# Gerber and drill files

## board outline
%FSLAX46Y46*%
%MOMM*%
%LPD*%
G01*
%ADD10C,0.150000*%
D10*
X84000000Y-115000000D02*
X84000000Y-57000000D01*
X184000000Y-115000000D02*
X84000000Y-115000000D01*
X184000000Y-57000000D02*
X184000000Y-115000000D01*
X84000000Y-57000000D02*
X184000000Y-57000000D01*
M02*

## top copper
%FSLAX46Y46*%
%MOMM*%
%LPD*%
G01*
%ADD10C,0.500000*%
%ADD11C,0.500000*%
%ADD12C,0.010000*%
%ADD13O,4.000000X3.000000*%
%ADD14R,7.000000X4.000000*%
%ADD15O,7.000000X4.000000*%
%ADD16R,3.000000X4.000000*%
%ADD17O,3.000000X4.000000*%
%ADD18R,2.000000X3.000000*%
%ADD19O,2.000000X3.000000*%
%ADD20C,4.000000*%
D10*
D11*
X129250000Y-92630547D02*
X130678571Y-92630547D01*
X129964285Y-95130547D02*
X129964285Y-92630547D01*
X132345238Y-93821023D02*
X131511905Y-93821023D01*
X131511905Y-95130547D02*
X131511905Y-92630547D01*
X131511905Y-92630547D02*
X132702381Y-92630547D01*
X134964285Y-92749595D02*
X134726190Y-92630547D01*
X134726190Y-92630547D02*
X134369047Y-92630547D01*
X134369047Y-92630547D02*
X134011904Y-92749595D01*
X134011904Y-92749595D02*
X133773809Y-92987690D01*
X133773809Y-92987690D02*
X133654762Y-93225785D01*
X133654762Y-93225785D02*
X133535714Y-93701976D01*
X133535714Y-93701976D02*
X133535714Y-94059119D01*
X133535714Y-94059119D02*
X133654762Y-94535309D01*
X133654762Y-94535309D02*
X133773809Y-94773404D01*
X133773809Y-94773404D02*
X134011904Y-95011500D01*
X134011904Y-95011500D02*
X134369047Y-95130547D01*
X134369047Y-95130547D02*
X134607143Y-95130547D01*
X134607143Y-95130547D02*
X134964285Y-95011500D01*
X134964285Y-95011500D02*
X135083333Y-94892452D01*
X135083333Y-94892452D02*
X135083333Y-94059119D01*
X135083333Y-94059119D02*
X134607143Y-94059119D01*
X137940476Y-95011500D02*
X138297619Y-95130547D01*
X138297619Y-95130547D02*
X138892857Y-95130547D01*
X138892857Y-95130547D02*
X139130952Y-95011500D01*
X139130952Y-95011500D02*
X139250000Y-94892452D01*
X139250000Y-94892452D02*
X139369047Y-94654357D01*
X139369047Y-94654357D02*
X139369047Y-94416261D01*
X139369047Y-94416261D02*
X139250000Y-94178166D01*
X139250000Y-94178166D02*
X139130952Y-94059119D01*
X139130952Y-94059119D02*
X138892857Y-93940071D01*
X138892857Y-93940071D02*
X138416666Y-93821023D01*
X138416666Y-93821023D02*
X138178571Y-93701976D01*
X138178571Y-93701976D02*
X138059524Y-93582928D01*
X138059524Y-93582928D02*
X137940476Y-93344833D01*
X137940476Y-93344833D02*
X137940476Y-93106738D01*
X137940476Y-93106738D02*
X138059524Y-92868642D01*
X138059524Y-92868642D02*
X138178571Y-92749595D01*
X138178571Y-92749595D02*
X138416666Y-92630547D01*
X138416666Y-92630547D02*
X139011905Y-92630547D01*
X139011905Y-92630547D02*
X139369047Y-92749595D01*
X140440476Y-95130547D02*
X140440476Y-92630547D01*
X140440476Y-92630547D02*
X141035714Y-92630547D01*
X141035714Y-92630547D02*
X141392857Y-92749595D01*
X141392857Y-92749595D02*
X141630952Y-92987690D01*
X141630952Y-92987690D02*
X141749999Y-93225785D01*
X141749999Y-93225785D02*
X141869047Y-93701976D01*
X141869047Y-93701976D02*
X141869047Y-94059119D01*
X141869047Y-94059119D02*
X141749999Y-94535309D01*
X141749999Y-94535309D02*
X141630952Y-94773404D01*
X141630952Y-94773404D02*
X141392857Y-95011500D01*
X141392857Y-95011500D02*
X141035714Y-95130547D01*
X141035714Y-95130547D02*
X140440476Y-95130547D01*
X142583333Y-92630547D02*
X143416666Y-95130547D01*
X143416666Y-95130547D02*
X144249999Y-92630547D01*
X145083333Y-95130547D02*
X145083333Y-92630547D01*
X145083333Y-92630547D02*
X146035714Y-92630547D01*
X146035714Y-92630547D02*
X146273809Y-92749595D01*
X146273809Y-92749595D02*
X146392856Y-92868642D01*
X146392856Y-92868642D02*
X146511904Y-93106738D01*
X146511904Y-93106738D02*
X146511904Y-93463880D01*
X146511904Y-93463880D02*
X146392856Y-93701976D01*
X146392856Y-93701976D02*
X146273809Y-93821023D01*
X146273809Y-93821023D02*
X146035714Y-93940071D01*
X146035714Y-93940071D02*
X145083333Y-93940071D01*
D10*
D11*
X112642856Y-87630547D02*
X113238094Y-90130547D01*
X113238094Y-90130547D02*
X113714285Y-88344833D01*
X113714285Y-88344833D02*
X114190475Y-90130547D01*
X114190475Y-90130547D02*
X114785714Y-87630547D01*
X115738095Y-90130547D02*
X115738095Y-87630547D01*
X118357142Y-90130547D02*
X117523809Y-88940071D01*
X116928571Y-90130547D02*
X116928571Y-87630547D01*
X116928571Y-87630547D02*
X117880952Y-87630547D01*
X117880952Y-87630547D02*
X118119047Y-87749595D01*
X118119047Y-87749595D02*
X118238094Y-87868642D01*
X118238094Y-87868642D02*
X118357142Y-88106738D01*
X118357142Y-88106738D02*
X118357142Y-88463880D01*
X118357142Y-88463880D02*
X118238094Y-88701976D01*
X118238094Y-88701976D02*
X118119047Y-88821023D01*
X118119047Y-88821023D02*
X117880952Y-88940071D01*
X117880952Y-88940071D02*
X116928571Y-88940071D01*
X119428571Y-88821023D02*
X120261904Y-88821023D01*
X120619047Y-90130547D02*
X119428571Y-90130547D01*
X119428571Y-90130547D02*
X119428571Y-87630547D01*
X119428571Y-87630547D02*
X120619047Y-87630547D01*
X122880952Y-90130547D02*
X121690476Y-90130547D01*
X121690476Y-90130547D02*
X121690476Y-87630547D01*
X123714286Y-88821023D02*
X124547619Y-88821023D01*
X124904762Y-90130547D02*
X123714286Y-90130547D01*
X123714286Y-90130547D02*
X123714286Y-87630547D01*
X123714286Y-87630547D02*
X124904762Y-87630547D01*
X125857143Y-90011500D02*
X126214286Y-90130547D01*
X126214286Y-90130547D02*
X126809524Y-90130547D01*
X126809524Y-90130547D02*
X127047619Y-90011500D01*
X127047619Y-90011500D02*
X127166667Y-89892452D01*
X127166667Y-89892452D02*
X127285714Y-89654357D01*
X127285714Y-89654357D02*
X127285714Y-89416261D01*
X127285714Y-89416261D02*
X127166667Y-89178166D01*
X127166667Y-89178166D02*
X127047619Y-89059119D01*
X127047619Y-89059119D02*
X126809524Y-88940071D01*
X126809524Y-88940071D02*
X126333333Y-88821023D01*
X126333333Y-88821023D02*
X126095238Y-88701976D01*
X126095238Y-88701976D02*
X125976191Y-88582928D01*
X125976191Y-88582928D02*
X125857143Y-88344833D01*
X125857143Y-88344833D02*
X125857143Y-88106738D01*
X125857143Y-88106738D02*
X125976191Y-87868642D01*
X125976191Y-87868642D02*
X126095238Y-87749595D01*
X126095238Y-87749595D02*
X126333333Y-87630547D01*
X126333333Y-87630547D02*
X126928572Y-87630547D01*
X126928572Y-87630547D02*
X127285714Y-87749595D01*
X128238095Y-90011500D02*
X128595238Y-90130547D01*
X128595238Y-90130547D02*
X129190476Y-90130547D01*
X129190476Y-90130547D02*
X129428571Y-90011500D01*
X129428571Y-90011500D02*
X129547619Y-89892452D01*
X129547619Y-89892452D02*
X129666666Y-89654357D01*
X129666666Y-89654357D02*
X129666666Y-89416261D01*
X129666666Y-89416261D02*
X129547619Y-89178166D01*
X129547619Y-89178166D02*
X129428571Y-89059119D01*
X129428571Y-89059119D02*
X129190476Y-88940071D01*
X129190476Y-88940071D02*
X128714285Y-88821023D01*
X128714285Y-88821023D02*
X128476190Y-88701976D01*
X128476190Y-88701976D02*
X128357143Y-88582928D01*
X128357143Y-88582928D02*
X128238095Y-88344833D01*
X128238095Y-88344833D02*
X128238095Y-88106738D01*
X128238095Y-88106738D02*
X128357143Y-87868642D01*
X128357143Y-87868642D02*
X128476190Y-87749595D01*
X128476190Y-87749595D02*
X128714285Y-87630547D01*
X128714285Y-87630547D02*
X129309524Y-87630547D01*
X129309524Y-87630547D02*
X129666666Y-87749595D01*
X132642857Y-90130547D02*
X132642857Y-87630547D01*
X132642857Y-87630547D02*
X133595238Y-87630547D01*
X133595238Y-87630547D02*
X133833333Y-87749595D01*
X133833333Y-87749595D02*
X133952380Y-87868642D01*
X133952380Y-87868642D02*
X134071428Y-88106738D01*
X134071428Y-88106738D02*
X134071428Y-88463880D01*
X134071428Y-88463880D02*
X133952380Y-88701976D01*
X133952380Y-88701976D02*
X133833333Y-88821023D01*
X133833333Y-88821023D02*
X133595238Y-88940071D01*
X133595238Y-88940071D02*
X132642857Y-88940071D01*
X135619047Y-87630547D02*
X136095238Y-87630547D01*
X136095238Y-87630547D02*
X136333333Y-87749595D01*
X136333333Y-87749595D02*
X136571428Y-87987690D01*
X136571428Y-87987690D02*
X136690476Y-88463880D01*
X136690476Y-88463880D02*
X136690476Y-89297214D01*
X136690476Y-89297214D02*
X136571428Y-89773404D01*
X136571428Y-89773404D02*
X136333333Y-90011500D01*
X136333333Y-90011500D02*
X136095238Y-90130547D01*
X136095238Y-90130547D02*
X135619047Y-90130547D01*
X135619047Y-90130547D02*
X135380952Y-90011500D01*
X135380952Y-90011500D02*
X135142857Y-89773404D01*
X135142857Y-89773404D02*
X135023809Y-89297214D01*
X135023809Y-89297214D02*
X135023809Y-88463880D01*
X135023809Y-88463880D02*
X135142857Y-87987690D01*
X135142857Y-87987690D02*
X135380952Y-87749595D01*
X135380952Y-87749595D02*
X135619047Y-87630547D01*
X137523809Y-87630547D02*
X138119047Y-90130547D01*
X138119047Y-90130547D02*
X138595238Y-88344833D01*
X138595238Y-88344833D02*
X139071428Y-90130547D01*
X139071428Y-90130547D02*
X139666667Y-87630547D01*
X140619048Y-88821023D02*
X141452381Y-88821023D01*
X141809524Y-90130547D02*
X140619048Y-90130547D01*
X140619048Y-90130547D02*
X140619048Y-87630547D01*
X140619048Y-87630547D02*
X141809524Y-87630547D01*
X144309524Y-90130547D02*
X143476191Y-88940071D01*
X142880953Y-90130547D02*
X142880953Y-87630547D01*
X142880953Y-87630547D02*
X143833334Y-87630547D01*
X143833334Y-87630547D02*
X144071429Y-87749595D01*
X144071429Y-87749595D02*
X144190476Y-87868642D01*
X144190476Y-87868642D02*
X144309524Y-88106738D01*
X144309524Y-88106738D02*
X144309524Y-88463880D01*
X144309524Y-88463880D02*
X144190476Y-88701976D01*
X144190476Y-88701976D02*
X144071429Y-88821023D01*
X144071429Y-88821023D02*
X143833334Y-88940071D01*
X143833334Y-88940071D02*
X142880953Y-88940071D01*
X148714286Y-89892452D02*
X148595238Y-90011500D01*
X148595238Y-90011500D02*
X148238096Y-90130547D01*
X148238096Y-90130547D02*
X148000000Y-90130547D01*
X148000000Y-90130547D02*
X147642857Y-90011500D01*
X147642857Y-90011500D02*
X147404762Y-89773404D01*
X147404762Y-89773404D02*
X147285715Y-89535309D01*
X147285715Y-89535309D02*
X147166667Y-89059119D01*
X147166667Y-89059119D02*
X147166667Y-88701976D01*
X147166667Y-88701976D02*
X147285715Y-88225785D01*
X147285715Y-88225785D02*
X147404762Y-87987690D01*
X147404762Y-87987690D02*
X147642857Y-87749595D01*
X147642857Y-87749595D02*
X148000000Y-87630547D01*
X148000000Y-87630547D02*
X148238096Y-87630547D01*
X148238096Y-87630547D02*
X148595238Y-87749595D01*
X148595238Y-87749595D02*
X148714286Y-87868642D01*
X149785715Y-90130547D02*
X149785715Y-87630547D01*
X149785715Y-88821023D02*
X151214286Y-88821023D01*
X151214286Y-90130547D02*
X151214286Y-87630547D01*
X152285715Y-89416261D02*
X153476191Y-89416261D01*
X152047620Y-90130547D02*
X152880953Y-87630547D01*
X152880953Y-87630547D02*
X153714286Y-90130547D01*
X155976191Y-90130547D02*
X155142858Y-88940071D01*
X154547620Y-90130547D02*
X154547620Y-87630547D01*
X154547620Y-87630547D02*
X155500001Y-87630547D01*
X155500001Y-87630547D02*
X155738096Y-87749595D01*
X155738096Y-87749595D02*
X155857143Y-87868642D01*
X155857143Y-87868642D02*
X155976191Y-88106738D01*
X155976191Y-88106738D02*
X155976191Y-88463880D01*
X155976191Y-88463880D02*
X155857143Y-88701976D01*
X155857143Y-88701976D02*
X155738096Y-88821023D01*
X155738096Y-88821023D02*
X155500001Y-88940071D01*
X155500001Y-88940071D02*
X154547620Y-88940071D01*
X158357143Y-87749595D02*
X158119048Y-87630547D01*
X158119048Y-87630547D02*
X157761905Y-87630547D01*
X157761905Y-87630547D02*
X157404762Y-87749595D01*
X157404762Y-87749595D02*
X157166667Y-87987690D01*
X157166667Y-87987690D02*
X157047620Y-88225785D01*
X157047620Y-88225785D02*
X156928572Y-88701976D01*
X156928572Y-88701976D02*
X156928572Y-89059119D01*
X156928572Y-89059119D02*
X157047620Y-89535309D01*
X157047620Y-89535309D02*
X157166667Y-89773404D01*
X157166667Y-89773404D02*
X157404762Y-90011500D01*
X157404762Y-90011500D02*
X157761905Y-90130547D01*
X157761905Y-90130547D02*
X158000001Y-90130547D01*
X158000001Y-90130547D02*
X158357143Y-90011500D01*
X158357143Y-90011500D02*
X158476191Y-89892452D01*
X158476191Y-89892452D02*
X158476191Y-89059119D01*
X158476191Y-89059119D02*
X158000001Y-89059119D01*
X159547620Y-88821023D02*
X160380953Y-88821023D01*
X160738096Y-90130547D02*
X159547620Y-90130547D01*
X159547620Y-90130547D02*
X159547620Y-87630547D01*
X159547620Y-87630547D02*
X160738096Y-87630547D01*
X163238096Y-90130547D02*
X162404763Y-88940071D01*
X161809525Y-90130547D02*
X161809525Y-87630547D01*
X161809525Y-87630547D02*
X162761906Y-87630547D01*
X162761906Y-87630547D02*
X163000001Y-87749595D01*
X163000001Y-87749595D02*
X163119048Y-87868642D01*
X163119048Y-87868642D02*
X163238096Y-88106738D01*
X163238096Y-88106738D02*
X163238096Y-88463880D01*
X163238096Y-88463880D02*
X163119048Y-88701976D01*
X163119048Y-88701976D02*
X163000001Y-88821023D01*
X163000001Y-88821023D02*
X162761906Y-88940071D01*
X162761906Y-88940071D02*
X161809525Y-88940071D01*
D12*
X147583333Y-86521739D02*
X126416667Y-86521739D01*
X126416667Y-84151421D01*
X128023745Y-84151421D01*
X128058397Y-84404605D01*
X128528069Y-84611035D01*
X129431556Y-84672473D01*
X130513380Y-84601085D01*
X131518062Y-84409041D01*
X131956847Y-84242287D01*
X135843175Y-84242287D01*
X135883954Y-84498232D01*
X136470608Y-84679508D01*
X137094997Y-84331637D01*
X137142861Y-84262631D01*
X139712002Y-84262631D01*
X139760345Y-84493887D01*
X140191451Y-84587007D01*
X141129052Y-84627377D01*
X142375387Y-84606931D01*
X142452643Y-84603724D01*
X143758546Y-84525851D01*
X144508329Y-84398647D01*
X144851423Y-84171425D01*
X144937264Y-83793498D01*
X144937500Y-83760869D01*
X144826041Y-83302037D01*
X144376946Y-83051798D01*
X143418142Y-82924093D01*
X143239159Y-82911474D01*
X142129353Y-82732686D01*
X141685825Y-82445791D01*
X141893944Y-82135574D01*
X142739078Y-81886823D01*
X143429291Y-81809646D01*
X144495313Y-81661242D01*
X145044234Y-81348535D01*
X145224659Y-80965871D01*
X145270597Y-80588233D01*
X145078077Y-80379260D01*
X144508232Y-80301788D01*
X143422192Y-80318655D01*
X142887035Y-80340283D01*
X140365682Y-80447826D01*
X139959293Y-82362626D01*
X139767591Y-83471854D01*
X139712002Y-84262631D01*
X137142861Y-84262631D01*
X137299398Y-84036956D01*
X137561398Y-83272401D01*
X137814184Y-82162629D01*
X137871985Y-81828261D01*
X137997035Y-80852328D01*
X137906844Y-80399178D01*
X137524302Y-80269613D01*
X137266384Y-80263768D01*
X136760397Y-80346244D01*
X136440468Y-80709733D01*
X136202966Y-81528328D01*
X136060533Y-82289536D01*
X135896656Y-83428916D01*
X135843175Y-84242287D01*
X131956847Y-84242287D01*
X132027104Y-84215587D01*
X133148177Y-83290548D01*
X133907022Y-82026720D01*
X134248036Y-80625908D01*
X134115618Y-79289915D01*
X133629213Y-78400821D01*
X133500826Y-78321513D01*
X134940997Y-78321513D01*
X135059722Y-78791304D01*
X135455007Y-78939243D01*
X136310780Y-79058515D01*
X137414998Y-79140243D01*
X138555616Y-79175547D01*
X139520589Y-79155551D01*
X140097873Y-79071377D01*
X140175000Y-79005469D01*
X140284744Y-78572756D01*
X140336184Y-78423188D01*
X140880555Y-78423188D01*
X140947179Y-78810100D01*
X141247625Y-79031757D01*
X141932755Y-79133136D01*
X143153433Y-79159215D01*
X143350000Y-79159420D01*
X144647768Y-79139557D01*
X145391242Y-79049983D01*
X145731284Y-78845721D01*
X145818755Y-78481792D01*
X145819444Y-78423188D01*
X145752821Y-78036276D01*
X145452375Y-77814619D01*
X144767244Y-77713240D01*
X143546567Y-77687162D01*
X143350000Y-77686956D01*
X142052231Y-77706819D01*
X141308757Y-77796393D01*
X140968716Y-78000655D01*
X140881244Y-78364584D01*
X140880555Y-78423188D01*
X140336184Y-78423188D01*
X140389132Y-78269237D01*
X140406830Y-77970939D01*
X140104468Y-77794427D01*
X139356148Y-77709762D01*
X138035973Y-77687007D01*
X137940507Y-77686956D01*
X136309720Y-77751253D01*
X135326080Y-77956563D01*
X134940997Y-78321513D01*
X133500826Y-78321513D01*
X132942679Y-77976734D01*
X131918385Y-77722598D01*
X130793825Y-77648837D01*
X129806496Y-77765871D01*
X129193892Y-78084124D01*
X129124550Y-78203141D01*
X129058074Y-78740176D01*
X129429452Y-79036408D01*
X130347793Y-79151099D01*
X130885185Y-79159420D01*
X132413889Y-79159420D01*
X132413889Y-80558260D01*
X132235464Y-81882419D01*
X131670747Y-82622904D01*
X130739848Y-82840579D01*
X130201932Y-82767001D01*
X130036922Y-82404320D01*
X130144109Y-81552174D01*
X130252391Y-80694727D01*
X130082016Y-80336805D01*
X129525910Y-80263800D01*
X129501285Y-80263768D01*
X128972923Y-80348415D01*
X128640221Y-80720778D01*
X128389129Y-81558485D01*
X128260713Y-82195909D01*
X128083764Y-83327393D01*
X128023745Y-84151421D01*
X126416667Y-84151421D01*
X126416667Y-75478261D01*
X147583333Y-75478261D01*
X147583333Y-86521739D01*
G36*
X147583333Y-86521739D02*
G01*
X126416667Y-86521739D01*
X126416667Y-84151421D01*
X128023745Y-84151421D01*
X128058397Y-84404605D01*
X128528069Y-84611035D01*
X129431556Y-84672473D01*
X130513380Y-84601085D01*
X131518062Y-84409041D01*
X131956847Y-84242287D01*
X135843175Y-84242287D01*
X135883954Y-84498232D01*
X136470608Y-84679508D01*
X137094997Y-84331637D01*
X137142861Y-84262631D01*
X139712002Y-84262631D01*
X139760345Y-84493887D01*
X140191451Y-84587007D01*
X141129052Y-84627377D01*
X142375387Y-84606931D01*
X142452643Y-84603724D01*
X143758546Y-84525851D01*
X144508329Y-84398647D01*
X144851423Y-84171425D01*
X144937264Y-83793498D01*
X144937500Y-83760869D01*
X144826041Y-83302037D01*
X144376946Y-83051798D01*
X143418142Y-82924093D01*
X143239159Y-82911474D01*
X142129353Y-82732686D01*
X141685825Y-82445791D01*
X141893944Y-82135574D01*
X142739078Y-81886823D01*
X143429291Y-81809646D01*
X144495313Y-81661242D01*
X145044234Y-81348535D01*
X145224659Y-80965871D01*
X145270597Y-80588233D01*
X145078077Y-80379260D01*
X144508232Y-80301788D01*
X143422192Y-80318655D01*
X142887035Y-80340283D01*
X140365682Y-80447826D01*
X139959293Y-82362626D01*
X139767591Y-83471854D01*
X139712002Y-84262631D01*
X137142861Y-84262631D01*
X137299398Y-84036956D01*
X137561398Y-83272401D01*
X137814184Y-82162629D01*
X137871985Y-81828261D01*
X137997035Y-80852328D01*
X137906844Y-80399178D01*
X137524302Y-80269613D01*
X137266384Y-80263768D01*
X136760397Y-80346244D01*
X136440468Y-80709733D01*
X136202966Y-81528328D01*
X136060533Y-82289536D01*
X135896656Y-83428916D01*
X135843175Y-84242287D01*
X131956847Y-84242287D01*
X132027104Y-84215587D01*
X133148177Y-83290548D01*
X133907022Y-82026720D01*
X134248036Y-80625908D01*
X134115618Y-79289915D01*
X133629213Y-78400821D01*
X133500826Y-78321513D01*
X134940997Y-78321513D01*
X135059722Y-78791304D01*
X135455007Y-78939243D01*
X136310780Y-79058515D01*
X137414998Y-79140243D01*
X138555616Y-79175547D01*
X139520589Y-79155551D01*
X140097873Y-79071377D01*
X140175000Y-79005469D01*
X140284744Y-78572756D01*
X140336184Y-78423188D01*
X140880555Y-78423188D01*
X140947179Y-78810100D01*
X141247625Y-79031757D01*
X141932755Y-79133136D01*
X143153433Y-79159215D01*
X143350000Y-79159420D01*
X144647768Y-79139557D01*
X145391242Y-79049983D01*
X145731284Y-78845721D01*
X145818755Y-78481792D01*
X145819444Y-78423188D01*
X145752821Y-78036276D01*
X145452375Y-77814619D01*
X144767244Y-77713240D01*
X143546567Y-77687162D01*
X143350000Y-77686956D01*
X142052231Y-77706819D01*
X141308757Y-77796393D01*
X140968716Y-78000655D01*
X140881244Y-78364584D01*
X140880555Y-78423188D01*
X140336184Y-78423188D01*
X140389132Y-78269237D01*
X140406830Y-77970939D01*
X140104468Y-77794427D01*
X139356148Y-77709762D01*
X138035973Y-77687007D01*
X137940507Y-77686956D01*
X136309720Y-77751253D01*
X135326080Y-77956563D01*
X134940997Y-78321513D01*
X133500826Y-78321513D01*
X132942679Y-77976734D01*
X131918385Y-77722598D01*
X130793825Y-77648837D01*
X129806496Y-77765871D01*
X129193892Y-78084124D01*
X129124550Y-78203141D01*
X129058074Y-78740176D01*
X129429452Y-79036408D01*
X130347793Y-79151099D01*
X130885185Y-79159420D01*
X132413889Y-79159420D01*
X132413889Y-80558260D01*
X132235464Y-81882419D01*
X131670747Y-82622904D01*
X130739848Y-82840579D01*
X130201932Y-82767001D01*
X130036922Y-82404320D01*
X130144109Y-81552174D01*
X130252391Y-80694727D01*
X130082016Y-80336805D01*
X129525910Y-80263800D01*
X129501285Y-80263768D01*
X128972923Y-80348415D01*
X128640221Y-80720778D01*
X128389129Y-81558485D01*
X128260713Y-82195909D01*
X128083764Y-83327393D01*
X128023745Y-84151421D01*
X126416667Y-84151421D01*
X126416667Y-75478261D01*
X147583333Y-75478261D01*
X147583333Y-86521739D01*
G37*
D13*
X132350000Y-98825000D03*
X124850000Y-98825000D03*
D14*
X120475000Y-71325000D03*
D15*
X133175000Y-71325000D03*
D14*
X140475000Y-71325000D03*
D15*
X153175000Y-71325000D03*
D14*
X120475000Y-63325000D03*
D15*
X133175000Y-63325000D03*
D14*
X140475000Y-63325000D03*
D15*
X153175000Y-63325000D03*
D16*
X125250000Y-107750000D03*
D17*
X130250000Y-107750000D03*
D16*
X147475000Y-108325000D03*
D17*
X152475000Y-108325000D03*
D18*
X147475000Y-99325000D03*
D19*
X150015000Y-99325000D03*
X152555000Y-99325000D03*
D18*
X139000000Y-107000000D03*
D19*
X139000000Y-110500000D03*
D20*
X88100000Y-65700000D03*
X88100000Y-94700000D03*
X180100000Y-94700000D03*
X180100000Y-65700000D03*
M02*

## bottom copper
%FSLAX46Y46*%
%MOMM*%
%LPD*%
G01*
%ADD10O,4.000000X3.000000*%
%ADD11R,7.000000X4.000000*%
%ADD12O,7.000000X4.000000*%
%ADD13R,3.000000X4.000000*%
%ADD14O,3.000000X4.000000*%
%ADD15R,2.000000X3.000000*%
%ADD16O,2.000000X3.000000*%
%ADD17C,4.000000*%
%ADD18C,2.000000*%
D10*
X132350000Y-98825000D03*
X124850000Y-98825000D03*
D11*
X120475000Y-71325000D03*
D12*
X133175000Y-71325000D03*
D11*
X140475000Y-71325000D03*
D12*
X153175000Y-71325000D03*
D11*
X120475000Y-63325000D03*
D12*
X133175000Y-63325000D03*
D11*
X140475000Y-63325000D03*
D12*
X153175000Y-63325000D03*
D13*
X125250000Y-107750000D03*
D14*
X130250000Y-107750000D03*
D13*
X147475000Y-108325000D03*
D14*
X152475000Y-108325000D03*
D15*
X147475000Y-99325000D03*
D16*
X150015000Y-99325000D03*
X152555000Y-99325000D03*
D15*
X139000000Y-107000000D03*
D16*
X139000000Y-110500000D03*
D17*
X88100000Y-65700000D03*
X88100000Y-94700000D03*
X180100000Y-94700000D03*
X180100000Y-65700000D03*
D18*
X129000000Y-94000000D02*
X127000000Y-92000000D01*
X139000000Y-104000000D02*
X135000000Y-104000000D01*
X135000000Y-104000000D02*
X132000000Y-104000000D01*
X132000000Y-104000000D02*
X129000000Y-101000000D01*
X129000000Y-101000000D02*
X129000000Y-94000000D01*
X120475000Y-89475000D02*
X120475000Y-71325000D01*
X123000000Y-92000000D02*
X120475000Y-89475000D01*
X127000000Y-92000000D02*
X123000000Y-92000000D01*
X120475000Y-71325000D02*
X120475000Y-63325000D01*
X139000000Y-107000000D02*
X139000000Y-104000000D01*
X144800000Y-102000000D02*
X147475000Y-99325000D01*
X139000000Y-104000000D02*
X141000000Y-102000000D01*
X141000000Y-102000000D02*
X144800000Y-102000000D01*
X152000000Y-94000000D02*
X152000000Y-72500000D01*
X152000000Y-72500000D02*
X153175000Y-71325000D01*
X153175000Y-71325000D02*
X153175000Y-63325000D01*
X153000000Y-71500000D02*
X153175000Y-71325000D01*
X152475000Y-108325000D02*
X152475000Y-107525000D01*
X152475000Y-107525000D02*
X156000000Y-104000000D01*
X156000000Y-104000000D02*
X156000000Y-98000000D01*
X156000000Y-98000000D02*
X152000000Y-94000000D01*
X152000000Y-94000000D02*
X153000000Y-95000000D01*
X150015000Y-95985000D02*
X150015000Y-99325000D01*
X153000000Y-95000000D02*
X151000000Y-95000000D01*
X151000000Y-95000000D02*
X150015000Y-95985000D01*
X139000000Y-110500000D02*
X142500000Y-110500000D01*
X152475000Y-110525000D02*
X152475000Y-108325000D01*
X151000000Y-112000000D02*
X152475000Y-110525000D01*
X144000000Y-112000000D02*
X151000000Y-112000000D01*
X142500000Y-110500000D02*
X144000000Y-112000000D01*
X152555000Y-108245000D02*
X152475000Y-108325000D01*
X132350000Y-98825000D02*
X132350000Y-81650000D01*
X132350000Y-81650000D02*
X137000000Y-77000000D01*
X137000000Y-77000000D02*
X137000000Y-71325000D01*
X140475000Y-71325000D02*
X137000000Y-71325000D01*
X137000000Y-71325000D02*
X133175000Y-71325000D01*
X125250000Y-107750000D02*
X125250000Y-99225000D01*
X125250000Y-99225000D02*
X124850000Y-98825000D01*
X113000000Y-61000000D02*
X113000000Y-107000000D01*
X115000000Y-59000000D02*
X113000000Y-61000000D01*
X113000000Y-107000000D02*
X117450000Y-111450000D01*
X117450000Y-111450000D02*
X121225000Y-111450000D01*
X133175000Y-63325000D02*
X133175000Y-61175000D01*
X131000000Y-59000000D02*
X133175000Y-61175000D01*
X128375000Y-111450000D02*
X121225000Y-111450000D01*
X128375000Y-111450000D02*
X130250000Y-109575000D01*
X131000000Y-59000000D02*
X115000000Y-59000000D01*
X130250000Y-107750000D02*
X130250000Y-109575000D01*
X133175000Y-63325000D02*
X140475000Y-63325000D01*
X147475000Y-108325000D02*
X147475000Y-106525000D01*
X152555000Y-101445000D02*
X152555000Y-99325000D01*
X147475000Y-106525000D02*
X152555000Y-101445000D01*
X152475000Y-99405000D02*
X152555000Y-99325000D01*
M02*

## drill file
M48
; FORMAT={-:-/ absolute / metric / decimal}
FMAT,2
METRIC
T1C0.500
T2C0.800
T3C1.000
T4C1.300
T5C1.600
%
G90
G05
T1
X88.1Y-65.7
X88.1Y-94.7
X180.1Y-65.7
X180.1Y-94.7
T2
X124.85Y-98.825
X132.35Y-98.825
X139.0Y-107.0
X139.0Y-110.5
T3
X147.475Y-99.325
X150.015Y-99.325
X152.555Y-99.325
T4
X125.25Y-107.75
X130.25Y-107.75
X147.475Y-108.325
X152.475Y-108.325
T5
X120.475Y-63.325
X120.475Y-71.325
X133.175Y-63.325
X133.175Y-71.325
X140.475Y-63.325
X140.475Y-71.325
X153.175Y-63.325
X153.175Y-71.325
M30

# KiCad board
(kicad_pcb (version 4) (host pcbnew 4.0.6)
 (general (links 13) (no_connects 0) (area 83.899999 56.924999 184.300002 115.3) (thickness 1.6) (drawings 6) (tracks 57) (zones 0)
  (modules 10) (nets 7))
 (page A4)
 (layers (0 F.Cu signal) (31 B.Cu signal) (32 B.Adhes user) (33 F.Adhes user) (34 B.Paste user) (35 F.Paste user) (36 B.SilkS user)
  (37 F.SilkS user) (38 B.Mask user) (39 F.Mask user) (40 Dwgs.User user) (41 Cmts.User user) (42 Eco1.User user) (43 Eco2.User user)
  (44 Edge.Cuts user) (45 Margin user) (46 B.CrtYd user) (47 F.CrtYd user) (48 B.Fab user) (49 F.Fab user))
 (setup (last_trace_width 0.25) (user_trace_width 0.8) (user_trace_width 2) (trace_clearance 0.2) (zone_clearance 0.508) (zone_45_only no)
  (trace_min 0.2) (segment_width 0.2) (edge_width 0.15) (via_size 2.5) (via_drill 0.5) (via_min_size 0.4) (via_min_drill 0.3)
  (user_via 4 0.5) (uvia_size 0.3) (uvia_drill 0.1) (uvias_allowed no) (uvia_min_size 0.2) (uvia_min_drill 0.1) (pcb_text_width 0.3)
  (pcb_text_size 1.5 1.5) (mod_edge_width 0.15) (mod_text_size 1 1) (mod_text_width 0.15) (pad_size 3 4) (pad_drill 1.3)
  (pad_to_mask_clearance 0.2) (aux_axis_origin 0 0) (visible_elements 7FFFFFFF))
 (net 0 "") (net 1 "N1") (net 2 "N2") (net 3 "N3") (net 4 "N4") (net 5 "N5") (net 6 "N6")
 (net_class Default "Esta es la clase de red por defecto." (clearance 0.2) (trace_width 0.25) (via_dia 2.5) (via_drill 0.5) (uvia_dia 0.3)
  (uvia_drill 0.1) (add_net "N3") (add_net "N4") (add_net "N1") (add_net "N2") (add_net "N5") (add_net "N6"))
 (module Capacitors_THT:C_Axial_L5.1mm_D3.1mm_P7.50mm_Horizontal (layer F.Cu) (at 132.35 98.825 180)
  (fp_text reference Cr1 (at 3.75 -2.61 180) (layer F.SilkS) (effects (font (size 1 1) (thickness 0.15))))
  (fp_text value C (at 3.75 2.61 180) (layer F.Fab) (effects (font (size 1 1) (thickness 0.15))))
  (pad 1 thru_hole oval (at 0 0 180) (size 4 3) (drill 0.8) (layers *.Cu *.Mask) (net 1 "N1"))
  (pad 2 thru_hole oval (at 7.5 0 180) (size 4 3) (drill 0.8) (layers *.Cu *.Mask) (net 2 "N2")))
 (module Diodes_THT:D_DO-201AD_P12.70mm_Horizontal (layer F.Cu) (at 120.475 71.325)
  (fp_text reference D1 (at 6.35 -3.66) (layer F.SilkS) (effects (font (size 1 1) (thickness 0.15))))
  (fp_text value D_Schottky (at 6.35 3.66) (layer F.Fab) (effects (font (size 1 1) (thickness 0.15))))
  (pad 1 thru_hole rect (at 0 0) (size 7 4) (drill 1.6) (layers *.Cu *.Mask) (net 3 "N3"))
  (pad 2 thru_hole oval (at 12.7 0) (size 7 4) (drill 1.6) (layers *.Cu *.Mask) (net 1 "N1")))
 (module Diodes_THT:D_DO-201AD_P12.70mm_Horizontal (layer F.Cu) (at 140.475 71.325)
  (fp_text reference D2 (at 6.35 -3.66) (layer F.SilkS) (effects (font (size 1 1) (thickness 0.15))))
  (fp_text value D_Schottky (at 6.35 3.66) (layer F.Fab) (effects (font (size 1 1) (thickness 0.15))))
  (pad 1 thru_hole rect (at 0 0) (size 7 4) (drill 1.6) (layers *.Cu *.Mask) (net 1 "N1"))
  (pad 2 thru_hole oval (at 12.7 0) (size 7 4) (drill 1.6) (layers *.Cu *.Mask) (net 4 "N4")))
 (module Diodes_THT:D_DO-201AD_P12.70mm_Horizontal (layer F.Cu) (at 120.475 63.325)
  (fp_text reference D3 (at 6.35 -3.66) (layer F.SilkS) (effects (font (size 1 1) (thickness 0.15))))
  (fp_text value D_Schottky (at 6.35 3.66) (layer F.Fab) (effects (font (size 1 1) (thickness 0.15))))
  (pad 1 thru_hole rect (at 0 0) (size 7 4) (drill 1.6) (layers *.Cu *.Mask) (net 3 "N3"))
  (pad 2 thru_hole oval (at 12.7 0) (size 7 4) (drill 1.6) (layers *.Cu *.Mask) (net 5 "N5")))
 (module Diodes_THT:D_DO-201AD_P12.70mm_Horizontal (layer F.Cu) (at 140.475 63.325)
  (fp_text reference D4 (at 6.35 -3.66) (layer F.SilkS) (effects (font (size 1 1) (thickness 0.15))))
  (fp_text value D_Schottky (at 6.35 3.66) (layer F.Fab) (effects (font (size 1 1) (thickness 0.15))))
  (pad 1 thru_hole rect (at 0 0) (size 7 4) (drill 1.6) (layers *.Cu *.Mask) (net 5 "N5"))
  (pad 2 thru_hole oval (at 12.7 0) (size 7 4) (drill 1.6) (layers *.Cu *.Mask) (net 4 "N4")))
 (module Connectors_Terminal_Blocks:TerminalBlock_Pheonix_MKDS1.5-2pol (layer F.Cu) (at 125.25 107.75)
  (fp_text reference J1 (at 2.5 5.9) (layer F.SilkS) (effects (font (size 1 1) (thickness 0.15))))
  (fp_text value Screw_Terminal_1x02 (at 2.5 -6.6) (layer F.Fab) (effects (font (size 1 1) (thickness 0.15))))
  (pad 1 thru_hole rect (at 0 0) (size 3 4) (drill 1.3) (layers *.Cu *.Mask) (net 2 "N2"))
  (pad 2 thru_hole oval (at 5 0) (size 3 4) (drill 1.3) (layers *.Cu *.Mask) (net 5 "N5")))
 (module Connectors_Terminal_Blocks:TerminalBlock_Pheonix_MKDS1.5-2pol (layer F.Cu) (at 147.475 108.325)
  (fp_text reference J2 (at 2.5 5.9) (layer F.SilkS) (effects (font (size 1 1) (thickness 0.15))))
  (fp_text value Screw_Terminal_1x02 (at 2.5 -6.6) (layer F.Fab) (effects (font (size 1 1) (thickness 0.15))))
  (pad 1 thru_hole rect (at 0 0) (size 3 4) (drill 1.3) (layers *.Cu *.Mask) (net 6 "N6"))
  (pad 2 thru_hole oval (at 5 0) (size 3 4) (drill 1.3) (layers *.Cu *.Mask) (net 4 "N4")))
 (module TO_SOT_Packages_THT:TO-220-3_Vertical (layer F.Cu) (at 147.475 99.325)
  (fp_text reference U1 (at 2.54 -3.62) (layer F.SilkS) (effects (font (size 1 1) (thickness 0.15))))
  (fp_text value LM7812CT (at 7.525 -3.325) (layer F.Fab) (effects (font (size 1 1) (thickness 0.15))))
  (pad 1 thru_hole rect (at 0 0) (size 2 3) (drill 1) (layers *.Cu *.Mask) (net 3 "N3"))
  (pad 2 thru_hole oval (at 2.54 0) (size 2 3) (drill 1) (layers *.Cu *.Mask) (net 4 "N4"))
  (pad 3 thru_hole oval (at 5.08 0) (size 2 3) (drill 1) (layers *.Cu *.Mask) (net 6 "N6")))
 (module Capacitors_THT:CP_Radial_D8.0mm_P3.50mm (layer F.Cu) (at 139 107 270)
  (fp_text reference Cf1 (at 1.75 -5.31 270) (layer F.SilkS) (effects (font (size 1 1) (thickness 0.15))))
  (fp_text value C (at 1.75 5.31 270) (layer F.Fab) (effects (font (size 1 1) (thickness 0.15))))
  (pad 1 thru_hole rect (at 0 0 270) (size 3 2) (drill 0.8) (layers *.Cu *.Mask) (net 3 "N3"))
  (pad 2 thru_hole oval (at 3.5 0 270) (size 3 2) (drill 0.8) (layers *.Cu *.Mask) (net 4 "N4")))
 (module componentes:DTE (layer F.Cu) (at 137 81)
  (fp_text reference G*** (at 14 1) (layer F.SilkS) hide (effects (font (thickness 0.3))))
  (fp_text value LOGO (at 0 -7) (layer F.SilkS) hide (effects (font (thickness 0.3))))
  (fp_poly
   (pts (xy 10.583333 5.521739) (xy -10.583333 5.521739) (xy -10.583333 3.151421) (xy -8.976255 3.151421) (xy -8.941603 3.404605)
    (xy -8.471931 3.611035) (xy -7.568444 3.672473) (xy -6.48662 3.601085) (xy -5.481938 3.409041) (xy -5.043153 3.242287)
    (xy -1.156825 3.242287) (xy -1.116046 3.498232) (xy -0.529392 3.679508) (xy 0.094997 3.331637) (xy 0.142861 3.262631)
    (xy 2.712002 3.262631) (xy 2.760345 3.493887) (xy 3.191451 3.587007) (xy 4.129052 3.627377) (xy 5.375387 3.606931)
    (xy 5.452643 3.603724) (xy 6.758546 3.525851) (xy 7.508329 3.398647) (xy 7.851423 3.171425) (xy 7.937264 2.793498) (xy 7.9375 2.760869)
    (xy 7.826041 2.302037) (xy 7.376946 2.051798) (xy 6.418142 1.924093) (xy 6.239159 1.911474) (xy 5.129353 1.732686)
    (xy 4.685825 1.445791) (xy 4.893944 1.135574) (xy 5.739078 0.886823) (xy 6.429291 0.809646) (xy 7.495313 0.661242)
    (xy 8.044234 0.348535) (xy 8.224659 -0.034129) (xy 8.270597 -0.411767) (xy 8.078077 -0.62074) (xy 7.508232 -0.698212)
    (xy 6.422192 -0.681345) (xy 5.887035 -0.659717) (xy 3.365682 -0.552174) (xy 2.959293 1.362626) (xy 2.767591 2.471854)
    (xy 2.712002 3.262631) (xy 0.142861 3.262631) (xy 0.299398 3.036956) (xy 0.561398 2.272401) (xy 0.814184 1.162629)
    (xy 0.871985 0.828261) (xy 0.997035 -0.147672) (xy 0.906844 -0.600822) (xy 0.524302 -0.730387) (xy 0.266384 -0.736232)
    (xy -0.239603 -0.653756) (xy -0.559532 -0.290267) (xy -0.797034 0.528328) (xy -0.939467 1.289536) (xy -1.103344 2.428916)
    (xy -1.156825 3.242287) (xy -5.043153 3.242287) (xy -4.972896 3.215587) (xy -3.851823 2.290548) (xy -3.092978 1.02672)
    (xy -2.751964 -0.374092) (xy -2.884382 -1.710085) (xy -3.370787 -2.599179) (xy -3.499174 -2.678487) (xy -2.059003 -2.678487)
    (xy -1.940278 -2.208696) (xy -1.544993 -2.060757) (xy -0.68922 -1.941485) (xy 0.414998 -1.859757) (xy 1.555616 -1.824453)
    (xy 2.520589 -1.844449) (xy 3.097873 -1.928623) (xy 3.175 -1.994531) (xy 3.284744 -2.427244) (xy 3.336184 -2.576812)
    (xy 3.880555 -2.576812) (xy 3.947179 -2.1899) (xy 4.247625 -1.968243) (xy 4.932755 -1.866864) (xy 6.153433 -1.840785) (xy 6.35 -1.84058)
    (xy 7.647768 -1.860443) (xy 8.391242 -1.950017) (xy 8.731284 -2.154279) (xy 8.818755 -2.518208) (xy 8.819444 -2.576812)
    (xy 8.752821 -2.963724) (xy 8.452375 -3.185381) (xy 7.767244 -3.28676) (xy 6.546567 -3.312838) (xy 6.35 -3.313044)
    (xy 5.052231 -3.293181) (xy 4.308757 -3.203607) (xy 3.968716 -2.999345) (xy 3.881244 -2.635416) (xy 3.880555 -2.576812)
    (xy 3.336184 -2.576812) (xy 3.389132 -2.730763) (xy 3.40683 -3.029061) (xy 3.104468 -3.205573) (xy 2.356148 -3.290238)
    (xy 1.035973 -3.312993) (xy 0.940507 -3.313044) (xy -0.69028 -3.248747) (xy -1.67392 -3.043437) (xy -2.059003 -2.678487)
    (xy -3.499174 -2.678487) (xy -4.057321 -3.023266) (xy -5.081615 -3.277402) (xy -6.206175 -3.351163) (xy -7.193504 -3.234129)
    (xy -7.806108 -2.915876) (xy -7.87545 -2.796859) (xy -7.941926 -2.259824) (xy -7.570548 -1.963592) (xy -6.652207 -1.848901)
    (xy -6.114815 -1.84058) (xy -4.586111 -1.84058) (xy -4.586111 -0.44174) (xy -4.764536 0.882419) (xy -5.329253 1.622904)
    (xy -6.260152 1.840579) (xy -6.798068 1.767001) (xy -6.963078 1.40432) (xy -6.855891 0.552174) (xy -6.747609 -0.305273)
    (xy -6.917984 -0.663195) (xy -7.47409 -0.7362) (xy -7.498715 -0.736232) (xy -8.027077 -0.651585) (xy -8.359779 -0.279222)
    (xy -8.610871 0.558485) (xy -8.739287 1.195909) (xy -8.916236 2.327393) (xy -8.976255 3.151421) (xy -10.583333 3.151421)
    (xy -10.583333 -5.521739) (xy 10.583333 -5.521739) (xy 10.583333 5.521739))
   (layer F.Cu) (width 0.01)))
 (gr_line (start 84 115) (end 84 57) (angle 90) (layer Edge.Cuts) (width 0.15))
 (gr_line (start 184 115) (end 84 115) (angle 90) (layer Edge.Cuts) (width 0.15))
 (gr_line (start 184 57) (end 184 115) (angle 90) (layer Edge.Cuts) (width 0.15))
 (gr_line (start 84 57) (end 184 57) (angle 90) (layer Edge.Cuts) (width 0.15))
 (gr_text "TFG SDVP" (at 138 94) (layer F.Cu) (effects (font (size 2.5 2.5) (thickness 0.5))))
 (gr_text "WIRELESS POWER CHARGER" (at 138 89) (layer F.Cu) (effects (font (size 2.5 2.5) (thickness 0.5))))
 (via (at 88.1 65.7) (size 4) (drill 0.5) (layers F.Cu B.Cu) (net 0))
 (via (at 88.1 94.7) (size 4) (drill 0.5) (layers F.Cu B.Cu) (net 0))
 (via (at 180.1 94.7) (size 4) (drill 0.5) (layers F.Cu B.Cu) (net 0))
 (via (at 180.1 65.7) (size 4) (drill 0.5) (layers F.Cu B.Cu) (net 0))
 (segment (start 129 94) (end 127 92) (width 2) (layer B.Cu) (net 3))
 (segment (start 139 104) (end 135 104) (width 2) (layer B.Cu) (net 3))
 (segment (start 135 104) (end 132 104) (width 2) (layer B.Cu) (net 3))
 (segment (start 132 104) (end 129 101) (width 2) (layer B.Cu) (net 3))
 (segment (start 129 101) (end 129 94) (width 2) (layer B.Cu) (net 3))
 (segment (start 120.475 89.475) (end 120.475 71.325) (width 2) (layer B.Cu) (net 3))
 (segment (start 123 92) (end 120.475 89.475) (width 2) (layer B.Cu) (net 3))
 (segment (start 127 92) (end 123 92) (width 2) (layer B.Cu) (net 3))
 (segment (start 120.475 71.325) (end 120.475 63.325) (width 2) (layer B.Cu) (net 3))
 (segment (start 139 107) (end 139 104) (width 2) (layer B.Cu) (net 3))
 (segment (start 144.8 102) (end 147.475 99.325) (width 2) (layer B.Cu) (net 3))
 (segment (start 139 104) (end 141 102) (width 2) (layer B.Cu) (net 3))
 (segment (start 141 102) (end 144.8 102) (width 2) (layer B.Cu) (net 3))
 (segment (start 152 94) (end 152 72.5) (width 2) (layer B.Cu) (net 4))
 (segment (start 152 72.5) (end 153.175 71.325) (width 2) (layer B.Cu) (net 4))
 (segment (start 153.175 71.325) (end 153.175 63.325) (width 2) (layer B.Cu) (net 4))
 (segment (start 153 71.5) (end 153.175 71.325) (width 2) (layer B.Cu) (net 4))
 (segment (start 152.475 108.325) (end 152.475 107.525) (width 2) (layer B.Cu) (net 4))
 (segment (start 152.475 107.525) (end 156 104) (width 2) (layer B.Cu) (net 4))
 (segment (start 156 104) (end 156 98) (width 2) (layer B.Cu) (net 4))
 (segment (start 156 98) (end 152 94) (width 2) (layer B.Cu) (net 4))
 (segment (start 152 94) (end 153 95) (width 2) (layer B.Cu) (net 4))
 (segment (start 150.015 95.985) (end 150.015 99.325) (width 2) (layer B.Cu) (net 4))
 (segment (start 153 95) (end 151 95) (width 2) (layer B.Cu) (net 4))
 (segment (start 151 95) (end 150.015 95.985) (width 2) (layer B.Cu) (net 4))
 (segment (start 139 110.5) (end 142.5 110.5) (width 2) (layer B.Cu) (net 4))
 (segment (start 152.475 110.525) (end 152.475 108.325) (width 2) (layer B.Cu) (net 4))
 (segment (start 151 112) (end 152.475 110.525) (width 2) (layer B.Cu) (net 4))
 (segment (start 144 112) (end 151 112) (width 2) (layer B.Cu) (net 4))
 (segment (start 142.5 110.5) (end 144 112) (width 2) (layer B.Cu) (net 4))
 (segment (start 152.555 108.245) (end 152.475 108.325) (width 2) (layer B.Cu) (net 4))
 (segment (start 132.35 98.825) (end 132.35 81.65) (width 2) (layer B.Cu) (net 1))
 (segment (start 132.35 81.65) (end 137 77) (width 2) (layer B.Cu) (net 1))
 (segment (start 137 77) (end 137 71.325) (width 2) (layer B.Cu) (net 1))
 (segment (start 140.475 71.325) (end 137 71.325) (width 2) (layer B.Cu) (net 1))
 (segment (start 137 71.325) (end 133.175 71.325) (width 2) (layer B.Cu) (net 1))
 (segment (start 125.25 107.75) (end 125.25 99.225) (width 2) (layer B.Cu) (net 2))
 (segment (start 125.25 99.225) (end 124.85 98.825) (width 2) (layer B.Cu) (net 2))
 (segment (start 113 61) (end 113 107) (width 2) (layer B.Cu) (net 5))
 (segment (start 115 59) (end 113 61) (width 2) (layer B.Cu) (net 5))
 (segment (start 113 107) (end 117.45 111.45) (width 2) (layer B.Cu) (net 5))
 (segment (start 117.45 111.45) (end 121.225 111.45) (width 2) (layer B.Cu) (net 5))
 (segment (start 133.175 63.325) (end 133.175 61.175) (width 2) (layer B.Cu) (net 5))
 (segment (start 131 59) (end 133.175 61.175) (width 2) (layer B.Cu) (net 5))
 (segment (start 128.375 111.45) (end 121.225 111.45) (width 2) (layer B.Cu) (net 5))
 (segment (start 128.375 111.45) (end 130.25 109.575) (width 2) (layer B.Cu) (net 5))
 (segment (start 131 59) (end 115 59) (width 2) (layer B.Cu) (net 5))
 (segment (start 130.25 107.75) (end 130.25 109.575) (width 2) (layer B.Cu) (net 5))
 (segment (start 133.175 63.325) (end 140.475 63.325) (width 2) (layer B.Cu) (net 5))
 (segment (start 147.475 108.325) (end 147.475 106.525) (width 2) (layer B.Cu) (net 6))
 (segment (start 152.555 101.445) (end 152.555 99.325) (width 2) (layer B.Cu) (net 6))
 (segment (start 147.475 106.525) (end 152.555 101.445) (width 2) (layer B.Cu) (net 6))
 (segment (start 152.475 99.405) (end 152.555 99.325) (width 2) (layer B.Cu) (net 6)))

